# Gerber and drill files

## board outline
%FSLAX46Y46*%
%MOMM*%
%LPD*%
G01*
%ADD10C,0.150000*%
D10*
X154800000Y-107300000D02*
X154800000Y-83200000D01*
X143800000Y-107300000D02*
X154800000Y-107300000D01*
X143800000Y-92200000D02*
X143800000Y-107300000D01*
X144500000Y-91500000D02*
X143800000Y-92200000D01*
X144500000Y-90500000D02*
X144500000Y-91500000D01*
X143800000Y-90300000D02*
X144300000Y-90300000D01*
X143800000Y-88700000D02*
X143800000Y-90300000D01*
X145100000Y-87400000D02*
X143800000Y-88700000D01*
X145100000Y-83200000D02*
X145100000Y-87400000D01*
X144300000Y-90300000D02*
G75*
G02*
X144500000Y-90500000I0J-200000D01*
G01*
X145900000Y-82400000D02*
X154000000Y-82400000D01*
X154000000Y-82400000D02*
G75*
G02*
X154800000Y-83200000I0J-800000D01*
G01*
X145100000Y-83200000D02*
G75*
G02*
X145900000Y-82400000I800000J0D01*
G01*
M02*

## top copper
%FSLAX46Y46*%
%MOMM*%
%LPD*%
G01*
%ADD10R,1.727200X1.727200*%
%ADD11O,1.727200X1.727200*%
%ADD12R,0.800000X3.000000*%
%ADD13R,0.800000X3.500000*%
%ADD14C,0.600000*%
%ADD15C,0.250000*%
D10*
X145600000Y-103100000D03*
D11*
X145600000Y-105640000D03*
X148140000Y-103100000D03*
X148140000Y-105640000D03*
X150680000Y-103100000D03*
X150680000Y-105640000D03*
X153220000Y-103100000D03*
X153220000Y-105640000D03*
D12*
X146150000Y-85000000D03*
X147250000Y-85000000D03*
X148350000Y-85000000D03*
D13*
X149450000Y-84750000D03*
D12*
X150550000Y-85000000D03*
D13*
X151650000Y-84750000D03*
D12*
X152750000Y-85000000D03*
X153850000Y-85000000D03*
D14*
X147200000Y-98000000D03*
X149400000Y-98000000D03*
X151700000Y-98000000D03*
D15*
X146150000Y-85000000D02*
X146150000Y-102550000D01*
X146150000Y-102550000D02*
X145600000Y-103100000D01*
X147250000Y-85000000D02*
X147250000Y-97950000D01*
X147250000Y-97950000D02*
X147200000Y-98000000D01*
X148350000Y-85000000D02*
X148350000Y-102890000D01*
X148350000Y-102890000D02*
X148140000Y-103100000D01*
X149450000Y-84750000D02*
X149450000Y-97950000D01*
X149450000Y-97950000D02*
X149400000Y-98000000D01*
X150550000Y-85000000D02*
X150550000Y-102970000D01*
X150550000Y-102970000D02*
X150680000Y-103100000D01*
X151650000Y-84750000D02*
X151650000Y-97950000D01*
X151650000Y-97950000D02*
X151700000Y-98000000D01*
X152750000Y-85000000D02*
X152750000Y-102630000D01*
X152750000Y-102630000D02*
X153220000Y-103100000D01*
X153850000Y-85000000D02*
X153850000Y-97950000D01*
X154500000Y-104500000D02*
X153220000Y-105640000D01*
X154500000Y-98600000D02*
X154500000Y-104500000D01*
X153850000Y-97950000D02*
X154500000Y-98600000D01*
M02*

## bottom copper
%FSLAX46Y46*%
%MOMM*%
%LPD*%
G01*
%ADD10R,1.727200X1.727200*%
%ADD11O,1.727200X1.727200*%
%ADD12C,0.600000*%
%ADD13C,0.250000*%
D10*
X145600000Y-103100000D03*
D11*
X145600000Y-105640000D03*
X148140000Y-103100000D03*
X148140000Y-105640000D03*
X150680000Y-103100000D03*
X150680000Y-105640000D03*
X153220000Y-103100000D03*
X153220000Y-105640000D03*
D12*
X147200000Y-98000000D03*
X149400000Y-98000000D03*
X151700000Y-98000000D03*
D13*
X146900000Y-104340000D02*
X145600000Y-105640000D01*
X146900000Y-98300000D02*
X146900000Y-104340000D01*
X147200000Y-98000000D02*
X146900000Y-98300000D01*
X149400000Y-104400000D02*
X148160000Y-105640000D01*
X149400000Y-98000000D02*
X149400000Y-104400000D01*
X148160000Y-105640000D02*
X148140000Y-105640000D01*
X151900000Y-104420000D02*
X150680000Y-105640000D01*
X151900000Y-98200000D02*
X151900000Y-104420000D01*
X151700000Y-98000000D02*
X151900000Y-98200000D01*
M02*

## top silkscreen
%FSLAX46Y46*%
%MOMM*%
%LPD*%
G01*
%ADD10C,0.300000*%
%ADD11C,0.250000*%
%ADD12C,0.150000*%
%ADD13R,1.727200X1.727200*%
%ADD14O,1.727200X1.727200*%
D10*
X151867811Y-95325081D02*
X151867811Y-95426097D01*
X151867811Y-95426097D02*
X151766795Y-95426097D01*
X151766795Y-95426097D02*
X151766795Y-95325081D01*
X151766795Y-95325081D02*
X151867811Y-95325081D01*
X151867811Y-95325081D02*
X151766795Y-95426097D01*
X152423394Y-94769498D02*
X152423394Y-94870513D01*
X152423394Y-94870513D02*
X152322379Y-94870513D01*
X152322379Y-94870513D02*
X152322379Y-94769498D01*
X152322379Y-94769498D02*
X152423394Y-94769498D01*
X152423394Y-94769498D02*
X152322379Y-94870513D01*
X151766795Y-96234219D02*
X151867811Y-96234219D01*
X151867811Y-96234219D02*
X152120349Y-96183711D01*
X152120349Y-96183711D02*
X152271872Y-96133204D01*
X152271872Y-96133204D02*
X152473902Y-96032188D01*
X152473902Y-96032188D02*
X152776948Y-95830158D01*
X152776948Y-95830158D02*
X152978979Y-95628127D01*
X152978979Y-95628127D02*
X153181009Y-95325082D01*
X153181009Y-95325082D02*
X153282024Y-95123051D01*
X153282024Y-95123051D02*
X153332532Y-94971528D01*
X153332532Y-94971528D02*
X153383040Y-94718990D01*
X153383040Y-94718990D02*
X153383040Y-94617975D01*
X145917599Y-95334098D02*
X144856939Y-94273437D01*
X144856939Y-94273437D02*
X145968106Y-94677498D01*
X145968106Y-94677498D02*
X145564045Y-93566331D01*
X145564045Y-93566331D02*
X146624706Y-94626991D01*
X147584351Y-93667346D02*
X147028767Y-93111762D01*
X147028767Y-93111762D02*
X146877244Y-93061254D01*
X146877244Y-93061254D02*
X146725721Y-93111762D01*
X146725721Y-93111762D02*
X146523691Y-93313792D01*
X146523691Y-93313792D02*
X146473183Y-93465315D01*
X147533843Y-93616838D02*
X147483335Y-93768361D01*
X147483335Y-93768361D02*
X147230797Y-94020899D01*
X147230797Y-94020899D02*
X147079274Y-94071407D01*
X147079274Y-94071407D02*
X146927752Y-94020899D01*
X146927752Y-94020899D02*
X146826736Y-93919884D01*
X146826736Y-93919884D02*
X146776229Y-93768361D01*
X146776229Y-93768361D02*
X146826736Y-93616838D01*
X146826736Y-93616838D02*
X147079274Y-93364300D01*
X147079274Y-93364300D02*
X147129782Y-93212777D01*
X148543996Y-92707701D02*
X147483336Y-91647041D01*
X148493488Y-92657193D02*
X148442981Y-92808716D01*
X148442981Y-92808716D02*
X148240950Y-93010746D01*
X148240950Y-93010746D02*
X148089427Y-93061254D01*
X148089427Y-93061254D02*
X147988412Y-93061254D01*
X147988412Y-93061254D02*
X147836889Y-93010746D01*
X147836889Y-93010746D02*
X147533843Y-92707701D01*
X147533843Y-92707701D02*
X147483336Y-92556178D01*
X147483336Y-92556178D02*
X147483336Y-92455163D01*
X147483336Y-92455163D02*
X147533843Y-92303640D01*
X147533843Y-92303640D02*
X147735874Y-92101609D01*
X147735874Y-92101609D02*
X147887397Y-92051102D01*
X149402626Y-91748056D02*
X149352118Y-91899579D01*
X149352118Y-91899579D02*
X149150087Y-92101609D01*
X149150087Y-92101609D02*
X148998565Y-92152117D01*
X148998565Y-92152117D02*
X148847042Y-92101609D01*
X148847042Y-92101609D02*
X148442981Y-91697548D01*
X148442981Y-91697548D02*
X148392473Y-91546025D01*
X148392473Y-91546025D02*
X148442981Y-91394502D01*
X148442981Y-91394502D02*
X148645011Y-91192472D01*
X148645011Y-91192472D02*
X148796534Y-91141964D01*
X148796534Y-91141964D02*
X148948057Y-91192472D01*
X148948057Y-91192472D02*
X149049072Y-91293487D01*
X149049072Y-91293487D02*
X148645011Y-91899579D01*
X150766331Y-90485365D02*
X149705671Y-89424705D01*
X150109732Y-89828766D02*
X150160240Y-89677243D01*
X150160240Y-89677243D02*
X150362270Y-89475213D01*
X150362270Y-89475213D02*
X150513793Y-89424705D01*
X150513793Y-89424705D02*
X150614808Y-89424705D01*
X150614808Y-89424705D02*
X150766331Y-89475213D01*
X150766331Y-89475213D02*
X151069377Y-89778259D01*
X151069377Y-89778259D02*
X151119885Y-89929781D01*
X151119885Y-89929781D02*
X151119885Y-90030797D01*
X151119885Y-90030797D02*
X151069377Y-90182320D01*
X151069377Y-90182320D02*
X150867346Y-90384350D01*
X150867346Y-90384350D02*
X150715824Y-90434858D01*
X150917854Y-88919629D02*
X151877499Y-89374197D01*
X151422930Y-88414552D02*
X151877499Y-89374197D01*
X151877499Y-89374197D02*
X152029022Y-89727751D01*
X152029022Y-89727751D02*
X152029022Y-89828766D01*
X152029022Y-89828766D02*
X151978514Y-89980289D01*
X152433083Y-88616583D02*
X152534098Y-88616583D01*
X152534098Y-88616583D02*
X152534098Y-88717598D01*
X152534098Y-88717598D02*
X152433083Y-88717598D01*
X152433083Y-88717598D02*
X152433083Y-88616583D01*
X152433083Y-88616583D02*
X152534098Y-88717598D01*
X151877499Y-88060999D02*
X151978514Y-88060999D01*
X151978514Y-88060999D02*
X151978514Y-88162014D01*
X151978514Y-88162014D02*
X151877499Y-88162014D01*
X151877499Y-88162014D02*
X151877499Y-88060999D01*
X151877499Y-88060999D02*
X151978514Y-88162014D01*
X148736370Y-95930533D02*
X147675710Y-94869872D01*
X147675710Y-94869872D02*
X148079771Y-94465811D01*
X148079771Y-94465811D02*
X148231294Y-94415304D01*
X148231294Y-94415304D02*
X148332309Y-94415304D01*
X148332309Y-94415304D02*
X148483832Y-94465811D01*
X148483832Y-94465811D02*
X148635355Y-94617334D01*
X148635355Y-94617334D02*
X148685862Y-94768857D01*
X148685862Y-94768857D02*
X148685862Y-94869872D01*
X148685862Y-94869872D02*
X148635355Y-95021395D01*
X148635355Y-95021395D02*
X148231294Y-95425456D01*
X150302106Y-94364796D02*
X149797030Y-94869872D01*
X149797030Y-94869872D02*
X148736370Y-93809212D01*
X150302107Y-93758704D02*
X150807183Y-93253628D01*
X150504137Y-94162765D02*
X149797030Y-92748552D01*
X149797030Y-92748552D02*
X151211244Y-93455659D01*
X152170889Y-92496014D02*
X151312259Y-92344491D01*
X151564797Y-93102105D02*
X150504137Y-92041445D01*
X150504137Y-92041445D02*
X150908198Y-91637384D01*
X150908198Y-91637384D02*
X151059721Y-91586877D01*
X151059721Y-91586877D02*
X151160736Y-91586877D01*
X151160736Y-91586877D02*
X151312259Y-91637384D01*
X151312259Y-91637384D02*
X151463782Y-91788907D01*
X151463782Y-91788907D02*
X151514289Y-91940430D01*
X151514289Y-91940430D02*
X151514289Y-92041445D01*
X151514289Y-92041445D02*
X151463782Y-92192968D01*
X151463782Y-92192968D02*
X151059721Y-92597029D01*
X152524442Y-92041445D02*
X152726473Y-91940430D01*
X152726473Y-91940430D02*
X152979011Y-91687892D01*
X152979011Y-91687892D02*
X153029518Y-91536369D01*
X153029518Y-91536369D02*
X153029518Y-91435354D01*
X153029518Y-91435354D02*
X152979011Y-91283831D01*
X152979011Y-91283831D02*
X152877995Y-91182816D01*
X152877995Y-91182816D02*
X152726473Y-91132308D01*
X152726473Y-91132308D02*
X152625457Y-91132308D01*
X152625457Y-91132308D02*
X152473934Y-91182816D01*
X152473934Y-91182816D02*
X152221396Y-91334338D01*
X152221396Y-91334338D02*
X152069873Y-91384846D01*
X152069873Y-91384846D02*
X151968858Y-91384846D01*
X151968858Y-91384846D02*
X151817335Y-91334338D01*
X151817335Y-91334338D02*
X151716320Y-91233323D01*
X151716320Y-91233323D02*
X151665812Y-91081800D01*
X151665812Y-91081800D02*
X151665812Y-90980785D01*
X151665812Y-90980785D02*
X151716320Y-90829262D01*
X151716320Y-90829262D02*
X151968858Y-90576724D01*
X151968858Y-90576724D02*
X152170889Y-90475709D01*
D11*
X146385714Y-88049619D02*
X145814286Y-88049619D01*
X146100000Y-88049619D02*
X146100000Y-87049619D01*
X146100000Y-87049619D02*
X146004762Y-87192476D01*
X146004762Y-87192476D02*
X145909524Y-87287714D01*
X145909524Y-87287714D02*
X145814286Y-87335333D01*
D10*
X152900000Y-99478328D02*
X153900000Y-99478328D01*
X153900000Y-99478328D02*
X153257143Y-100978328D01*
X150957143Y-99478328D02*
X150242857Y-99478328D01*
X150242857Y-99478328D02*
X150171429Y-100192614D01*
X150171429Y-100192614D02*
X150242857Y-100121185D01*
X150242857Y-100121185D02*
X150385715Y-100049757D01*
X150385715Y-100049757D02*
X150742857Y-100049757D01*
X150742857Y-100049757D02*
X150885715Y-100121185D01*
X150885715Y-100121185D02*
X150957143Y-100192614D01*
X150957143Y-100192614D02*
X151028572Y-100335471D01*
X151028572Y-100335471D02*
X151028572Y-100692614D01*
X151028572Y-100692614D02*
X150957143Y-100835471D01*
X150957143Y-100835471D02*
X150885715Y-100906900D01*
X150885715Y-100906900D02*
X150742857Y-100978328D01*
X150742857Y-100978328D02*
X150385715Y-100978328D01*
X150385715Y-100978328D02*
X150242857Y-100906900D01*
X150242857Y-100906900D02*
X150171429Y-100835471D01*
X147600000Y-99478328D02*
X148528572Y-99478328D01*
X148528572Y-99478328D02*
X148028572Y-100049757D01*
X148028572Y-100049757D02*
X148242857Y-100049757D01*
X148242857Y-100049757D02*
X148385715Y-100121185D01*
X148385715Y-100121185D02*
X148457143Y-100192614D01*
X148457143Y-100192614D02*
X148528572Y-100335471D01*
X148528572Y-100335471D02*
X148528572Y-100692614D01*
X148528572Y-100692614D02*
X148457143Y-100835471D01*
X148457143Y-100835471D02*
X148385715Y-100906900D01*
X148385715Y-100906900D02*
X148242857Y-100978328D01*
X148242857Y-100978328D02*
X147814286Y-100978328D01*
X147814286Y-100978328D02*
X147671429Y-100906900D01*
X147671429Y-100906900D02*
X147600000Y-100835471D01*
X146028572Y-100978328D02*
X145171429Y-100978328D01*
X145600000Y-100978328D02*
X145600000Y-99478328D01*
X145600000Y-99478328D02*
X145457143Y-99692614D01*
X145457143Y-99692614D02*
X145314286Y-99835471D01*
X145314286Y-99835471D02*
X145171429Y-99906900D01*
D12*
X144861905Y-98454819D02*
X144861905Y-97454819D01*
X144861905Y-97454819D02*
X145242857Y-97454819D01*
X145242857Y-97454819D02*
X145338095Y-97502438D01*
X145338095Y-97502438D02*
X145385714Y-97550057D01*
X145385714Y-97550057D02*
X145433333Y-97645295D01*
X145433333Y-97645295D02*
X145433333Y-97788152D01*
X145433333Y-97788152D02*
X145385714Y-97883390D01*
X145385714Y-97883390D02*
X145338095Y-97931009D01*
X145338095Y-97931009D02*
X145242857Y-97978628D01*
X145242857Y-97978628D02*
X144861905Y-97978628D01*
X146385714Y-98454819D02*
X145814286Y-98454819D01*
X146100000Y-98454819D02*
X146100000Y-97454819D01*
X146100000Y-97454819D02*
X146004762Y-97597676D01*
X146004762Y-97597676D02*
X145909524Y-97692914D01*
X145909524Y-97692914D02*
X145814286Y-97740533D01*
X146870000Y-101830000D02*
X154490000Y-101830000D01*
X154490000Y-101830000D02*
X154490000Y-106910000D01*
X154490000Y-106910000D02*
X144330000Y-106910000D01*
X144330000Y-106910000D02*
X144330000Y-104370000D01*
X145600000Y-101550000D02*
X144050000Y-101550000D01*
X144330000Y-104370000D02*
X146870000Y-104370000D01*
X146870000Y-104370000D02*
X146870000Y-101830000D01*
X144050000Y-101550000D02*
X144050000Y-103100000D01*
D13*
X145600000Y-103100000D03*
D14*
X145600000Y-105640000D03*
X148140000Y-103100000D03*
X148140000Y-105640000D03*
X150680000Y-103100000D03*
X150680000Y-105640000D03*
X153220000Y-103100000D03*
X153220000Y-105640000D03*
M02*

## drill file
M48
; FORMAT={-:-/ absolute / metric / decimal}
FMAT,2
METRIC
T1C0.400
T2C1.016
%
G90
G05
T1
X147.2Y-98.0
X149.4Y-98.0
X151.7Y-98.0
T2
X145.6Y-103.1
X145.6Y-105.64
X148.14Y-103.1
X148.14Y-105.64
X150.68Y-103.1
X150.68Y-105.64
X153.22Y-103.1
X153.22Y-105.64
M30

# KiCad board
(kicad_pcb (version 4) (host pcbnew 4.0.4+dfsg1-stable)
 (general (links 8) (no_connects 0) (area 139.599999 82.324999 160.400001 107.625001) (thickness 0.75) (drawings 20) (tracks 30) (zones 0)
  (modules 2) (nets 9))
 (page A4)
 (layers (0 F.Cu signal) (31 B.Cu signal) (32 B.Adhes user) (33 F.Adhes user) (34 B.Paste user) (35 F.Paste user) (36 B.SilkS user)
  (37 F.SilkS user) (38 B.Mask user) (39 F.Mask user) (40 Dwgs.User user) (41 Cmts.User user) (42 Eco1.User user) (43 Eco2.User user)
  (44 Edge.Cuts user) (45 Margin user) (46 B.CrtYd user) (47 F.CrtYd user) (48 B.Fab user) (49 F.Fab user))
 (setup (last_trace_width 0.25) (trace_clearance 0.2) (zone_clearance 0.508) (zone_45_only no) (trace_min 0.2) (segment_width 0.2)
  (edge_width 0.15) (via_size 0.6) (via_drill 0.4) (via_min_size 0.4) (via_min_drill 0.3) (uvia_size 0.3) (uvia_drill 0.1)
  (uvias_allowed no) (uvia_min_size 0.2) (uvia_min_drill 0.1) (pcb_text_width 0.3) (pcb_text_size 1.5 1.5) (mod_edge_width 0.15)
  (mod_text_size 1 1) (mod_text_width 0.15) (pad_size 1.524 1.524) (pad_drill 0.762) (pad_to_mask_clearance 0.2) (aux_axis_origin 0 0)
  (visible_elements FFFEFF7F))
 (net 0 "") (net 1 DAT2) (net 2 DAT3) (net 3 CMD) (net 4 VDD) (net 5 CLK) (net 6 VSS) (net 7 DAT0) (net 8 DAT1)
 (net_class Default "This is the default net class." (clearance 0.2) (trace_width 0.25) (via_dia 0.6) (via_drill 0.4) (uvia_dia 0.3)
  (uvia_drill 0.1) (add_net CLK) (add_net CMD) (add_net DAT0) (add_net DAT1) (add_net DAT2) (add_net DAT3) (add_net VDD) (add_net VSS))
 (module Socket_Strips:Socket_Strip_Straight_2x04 (layer F.Cu) (at 145.6 103.1)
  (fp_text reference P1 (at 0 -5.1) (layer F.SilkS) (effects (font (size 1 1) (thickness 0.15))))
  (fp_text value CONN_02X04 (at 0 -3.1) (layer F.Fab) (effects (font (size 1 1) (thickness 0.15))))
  (fp_line (start 1.27 -1.27) (end 8.89 -1.27) (layer F.SilkS) (width 0.15))
  (fp_line (start 8.89 -1.27) (end 8.89 3.81) (layer F.SilkS) (width 0.15))
  (fp_line (start 8.89 3.81) (end -1.27 3.81) (layer F.SilkS) (width 0.15))
  (fp_line (start -1.27 3.81) (end -1.27 1.27) (layer F.SilkS) (width 0.15))
  (fp_line (start 0 -1.55) (end -1.55 -1.55) (layer F.SilkS) (width 0.15))
  (fp_line (start -1.27 1.27) (end 1.27 1.27) (layer F.SilkS) (width 0.15))
  (fp_line (start 1.27 1.27) (end 1.27 -1.27) (layer F.SilkS) (width 0.15))
  (fp_line (start -1.55 -1.55) (end -1.55 0) (layer F.SilkS) (width 0.15))
  (pad 1 thru_hole rect (at 0 0) (size 1.7272 1.7272) (drill 1.016) (layers *.Cu *.Mask F.SilkS) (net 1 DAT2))
  (pad 2 thru_hole oval (at 0 2.54) (size 1.7272 1.7272) (drill 1.016) (layers *.Cu *.Mask F.SilkS) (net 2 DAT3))
  (pad 3 thru_hole oval (at 2.54 0) (size 1.7272 1.7272) (drill 1.016) (layers *.Cu *.Mask F.SilkS) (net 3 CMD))
  (pad 4 thru_hole oval (at 2.54 2.54) (size 1.7272 1.7272) (drill 1.016) (layers *.Cu *.Mask F.SilkS) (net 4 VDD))
  (pad 5 thru_hole oval (at 5.08 0) (size 1.7272 1.7272) (drill 1.016) (layers *.Cu *.Mask F.SilkS) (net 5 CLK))
  (pad 6 thru_hole oval (at 5.08 2.54) (size 1.7272 1.7272) (drill 1.016) (layers *.Cu *.Mask F.SilkS) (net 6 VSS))
  (pad 7 thru_hole oval (at 7.62 0) (size 1.7272 1.7272) (drill 1.016) (layers *.Cu *.Mask F.SilkS) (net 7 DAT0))
  (pad 8 thru_hole oval (at 7.62 2.54) (size 1.7272 1.7272) (drill 1.016) (layers *.Cu *.Mask F.SilkS) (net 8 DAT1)))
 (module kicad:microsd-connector (layer F.Cu) (at 150 85)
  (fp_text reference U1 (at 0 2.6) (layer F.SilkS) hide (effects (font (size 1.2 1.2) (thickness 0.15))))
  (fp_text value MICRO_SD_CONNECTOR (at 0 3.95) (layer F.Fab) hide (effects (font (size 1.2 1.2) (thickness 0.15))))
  (pad 1 smd rect (at -3.85 0) (size 0.8 3) (layers F.Cu F.Paste F.Mask) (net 1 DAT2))
  (pad 2 smd rect (at -2.75 0) (size 0.8 3) (layers F.Cu F.Paste F.Mask) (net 2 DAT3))
  (pad 3 smd rect (at -1.65 0) (size 0.8 3) (layers F.Cu F.Paste F.Mask) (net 3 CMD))
  (pad 4 smd rect (at -0.55 -0.25) (size 0.8 3.5) (layers F.Cu F.Paste F.Mask) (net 4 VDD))
  (pad 5 smd rect (at 0.55 0) (size 0.8 3) (layers F.Cu F.Paste F.Mask) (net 5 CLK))
  (pad 6 smd rect (at 1.65 -0.25) (size 0.8 3.5) (layers F.Cu F.Paste F.Mask) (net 6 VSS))
  (pad 7 smd rect (at 2.75 0) (size 0.8 3) (layers F.Cu F.Paste F.Mask) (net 7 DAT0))
  (pad 8 smd rect (at 3.85 0) (size 0.8 3) (layers F.Cu F.Paste F.Mask) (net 8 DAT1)))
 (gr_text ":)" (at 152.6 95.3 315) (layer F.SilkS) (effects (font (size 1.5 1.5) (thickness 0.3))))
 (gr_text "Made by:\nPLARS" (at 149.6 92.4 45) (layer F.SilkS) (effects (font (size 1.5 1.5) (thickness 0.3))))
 (gr_line (start 154.8 107.3) (end 154.8 83.2) (angle 90) (layer Edge.Cuts) (width 0.15))
 (gr_line (start 143.8 107.3) (end 154.8 107.3) (angle 90) (layer Edge.Cuts) (width 0.15))
 (gr_line (start 143.8 92.2) (end 143.8 107.3) (angle 90) (layer Edge.Cuts) (width 0.15))
 (gr_line (start 144.5 91.5) (end 143.8 92.2) (angle 90) (layer Edge.Cuts) (width 0.15))
 (gr_line (start 144.5 90.5) (end 144.5 91.5) (angle 90) (layer Edge.Cuts) (width 0.15))
 (gr_line (start 143.8 90.3) (end 144.3 90.3) (angle 90) (layer Edge.Cuts) (width 0.15))
 (gr_line (start 143.8 88.7) (end 143.8 90.3) (angle 90) (layer Edge.Cuts) (width 0.15))
 (gr_line (start 145.1 87.4) (end 143.8 88.7) (angle 90) (layer Edge.Cuts) (width 0.15))
 (gr_line (start 145.1 83.2) (end 145.1 87.4) (angle 90) (layer Edge.Cuts) (width 0.15))
 (gr_arc (start 144.3 90.5) (end 144.3 90.3) (angle 90) (layer Edge.Cuts) (width 0.15))
 (gr_line (start 145.9 82.4) (end 154 82.4) (angle 90) (layer Edge.Cuts) (width 0.15))
 (gr_arc (start 154 83.2) (end 154 82.4) (angle 90) (layer Edge.Cuts) (width 0.15))
 (gr_arc (start 145.9 83.2) (end 145.1 83.2) (angle 90) (layer Edge.Cuts) (width 0.15))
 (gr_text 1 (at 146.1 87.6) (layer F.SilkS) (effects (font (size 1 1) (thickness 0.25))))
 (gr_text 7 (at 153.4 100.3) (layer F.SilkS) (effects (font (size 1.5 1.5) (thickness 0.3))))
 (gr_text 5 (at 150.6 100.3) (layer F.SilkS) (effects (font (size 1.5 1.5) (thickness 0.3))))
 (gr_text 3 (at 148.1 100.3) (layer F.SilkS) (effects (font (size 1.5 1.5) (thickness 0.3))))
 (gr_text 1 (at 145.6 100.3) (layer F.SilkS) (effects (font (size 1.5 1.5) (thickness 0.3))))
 (segment (start 146.15 85) (end 146.15 102.55) (width 0.25) (layer F.Cu) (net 1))
 (segment (start 146.15 102.55) (end 145.6 103.1) (width 0.25) (layer F.Cu) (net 1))
 (segment (start 147.25 85) (end 147.25 97.95) (width 0.25) (layer F.Cu) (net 2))
 (segment (start 146.9 104.34) (end 145.6 105.64) (width 0.25) (layer B.Cu) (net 2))
 (segment (start 146.9 98.3) (end 146.9 104.34) (width 0.25) (layer B.Cu) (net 2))
 (segment (start 147.2 98) (end 146.9 98.3) (width 0.25) (layer B.Cu) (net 2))
 (via (at 147.2 98) (size 0.6) (drill 0.4) (layers F.Cu B.Cu) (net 2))
 (segment (start 147.25 97.95) (end 147.2 98) (width 0.25) (layer F.Cu) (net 2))
 (segment (start 148.35 85) (end 148.35 102.89) (width 0.25) (layer F.Cu) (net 3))
 (segment (start 148.35 102.89) (end 148.14 103.1) (width 0.25) (layer F.Cu) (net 3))
 (segment (start 149.45 84.75) (end 149.45 97.95) (width 0.25) (layer F.Cu) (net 4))
 (segment (start 149.4 104.4) (end 148.16 105.64) (width 0.25) (layer B.Cu) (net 4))
 (segment (start 149.4 98) (end 149.4 104.4) (width 0.25) (layer B.Cu) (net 4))
 (via (at 149.4 98) (size 0.6) (drill 0.4) (layers F.Cu B.Cu) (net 4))
 (segment (start 149.45 97.95) (end 149.4 98) (width 0.25) (layer F.Cu) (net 4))
 (segment (start 148.16 105.64) (end 148.14 105.64) (width 0.25) (layer B.Cu) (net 4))
 (segment (start 150.55 85) (end 150.55 102.97) (width 0.25) (layer F.Cu) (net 5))
 (segment (start 150.55 102.97) (end 150.68 103.1) (width 0.25) (layer F.Cu) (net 5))
 (segment (start 151.65 84.75) (end 151.65 97.95) (width 0.25) (layer F.Cu) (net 6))
 (segment (start 151.9 104.42) (end 150.68 105.64) (width 0.25) (layer B.Cu) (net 6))
 (segment (start 151.9 98.2) (end 151.9 104.42) (width 0.25) (layer B.Cu) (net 6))
 (segment (start 151.7 98) (end 151.9 98.2) (width 0.25) (layer B.Cu) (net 6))
 (via (at 151.7 98) (size 0.6) (drill 0.4) (layers F.Cu B.Cu) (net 6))
 (segment (start 151.65 97.95) (end 151.7 98) (width 0.25) (layer F.Cu) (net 6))
 (segment (start 152.75 85) (end 152.75 102.63) (width 0.25) (layer F.Cu) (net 7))
 (segment (start 152.75 102.63) (end 153.22 103.1) (width 0.25) (layer F.Cu) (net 7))
 (segment (start 153.85 85) (end 153.85 97.95) (width 0.25) (layer F.Cu) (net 8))
 (segment (start 154.5 104.5) (end 153.22 105.64) (width 0.25) (layer F.Cu) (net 8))
 (segment (start 154.5 98.6) (end 154.5 104.5) (width 0.25) (layer F.Cu) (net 8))
 (segment (start 153.85 97.95) (end 154.5 98.6) (width 0.25) (layer F.Cu) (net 8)))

